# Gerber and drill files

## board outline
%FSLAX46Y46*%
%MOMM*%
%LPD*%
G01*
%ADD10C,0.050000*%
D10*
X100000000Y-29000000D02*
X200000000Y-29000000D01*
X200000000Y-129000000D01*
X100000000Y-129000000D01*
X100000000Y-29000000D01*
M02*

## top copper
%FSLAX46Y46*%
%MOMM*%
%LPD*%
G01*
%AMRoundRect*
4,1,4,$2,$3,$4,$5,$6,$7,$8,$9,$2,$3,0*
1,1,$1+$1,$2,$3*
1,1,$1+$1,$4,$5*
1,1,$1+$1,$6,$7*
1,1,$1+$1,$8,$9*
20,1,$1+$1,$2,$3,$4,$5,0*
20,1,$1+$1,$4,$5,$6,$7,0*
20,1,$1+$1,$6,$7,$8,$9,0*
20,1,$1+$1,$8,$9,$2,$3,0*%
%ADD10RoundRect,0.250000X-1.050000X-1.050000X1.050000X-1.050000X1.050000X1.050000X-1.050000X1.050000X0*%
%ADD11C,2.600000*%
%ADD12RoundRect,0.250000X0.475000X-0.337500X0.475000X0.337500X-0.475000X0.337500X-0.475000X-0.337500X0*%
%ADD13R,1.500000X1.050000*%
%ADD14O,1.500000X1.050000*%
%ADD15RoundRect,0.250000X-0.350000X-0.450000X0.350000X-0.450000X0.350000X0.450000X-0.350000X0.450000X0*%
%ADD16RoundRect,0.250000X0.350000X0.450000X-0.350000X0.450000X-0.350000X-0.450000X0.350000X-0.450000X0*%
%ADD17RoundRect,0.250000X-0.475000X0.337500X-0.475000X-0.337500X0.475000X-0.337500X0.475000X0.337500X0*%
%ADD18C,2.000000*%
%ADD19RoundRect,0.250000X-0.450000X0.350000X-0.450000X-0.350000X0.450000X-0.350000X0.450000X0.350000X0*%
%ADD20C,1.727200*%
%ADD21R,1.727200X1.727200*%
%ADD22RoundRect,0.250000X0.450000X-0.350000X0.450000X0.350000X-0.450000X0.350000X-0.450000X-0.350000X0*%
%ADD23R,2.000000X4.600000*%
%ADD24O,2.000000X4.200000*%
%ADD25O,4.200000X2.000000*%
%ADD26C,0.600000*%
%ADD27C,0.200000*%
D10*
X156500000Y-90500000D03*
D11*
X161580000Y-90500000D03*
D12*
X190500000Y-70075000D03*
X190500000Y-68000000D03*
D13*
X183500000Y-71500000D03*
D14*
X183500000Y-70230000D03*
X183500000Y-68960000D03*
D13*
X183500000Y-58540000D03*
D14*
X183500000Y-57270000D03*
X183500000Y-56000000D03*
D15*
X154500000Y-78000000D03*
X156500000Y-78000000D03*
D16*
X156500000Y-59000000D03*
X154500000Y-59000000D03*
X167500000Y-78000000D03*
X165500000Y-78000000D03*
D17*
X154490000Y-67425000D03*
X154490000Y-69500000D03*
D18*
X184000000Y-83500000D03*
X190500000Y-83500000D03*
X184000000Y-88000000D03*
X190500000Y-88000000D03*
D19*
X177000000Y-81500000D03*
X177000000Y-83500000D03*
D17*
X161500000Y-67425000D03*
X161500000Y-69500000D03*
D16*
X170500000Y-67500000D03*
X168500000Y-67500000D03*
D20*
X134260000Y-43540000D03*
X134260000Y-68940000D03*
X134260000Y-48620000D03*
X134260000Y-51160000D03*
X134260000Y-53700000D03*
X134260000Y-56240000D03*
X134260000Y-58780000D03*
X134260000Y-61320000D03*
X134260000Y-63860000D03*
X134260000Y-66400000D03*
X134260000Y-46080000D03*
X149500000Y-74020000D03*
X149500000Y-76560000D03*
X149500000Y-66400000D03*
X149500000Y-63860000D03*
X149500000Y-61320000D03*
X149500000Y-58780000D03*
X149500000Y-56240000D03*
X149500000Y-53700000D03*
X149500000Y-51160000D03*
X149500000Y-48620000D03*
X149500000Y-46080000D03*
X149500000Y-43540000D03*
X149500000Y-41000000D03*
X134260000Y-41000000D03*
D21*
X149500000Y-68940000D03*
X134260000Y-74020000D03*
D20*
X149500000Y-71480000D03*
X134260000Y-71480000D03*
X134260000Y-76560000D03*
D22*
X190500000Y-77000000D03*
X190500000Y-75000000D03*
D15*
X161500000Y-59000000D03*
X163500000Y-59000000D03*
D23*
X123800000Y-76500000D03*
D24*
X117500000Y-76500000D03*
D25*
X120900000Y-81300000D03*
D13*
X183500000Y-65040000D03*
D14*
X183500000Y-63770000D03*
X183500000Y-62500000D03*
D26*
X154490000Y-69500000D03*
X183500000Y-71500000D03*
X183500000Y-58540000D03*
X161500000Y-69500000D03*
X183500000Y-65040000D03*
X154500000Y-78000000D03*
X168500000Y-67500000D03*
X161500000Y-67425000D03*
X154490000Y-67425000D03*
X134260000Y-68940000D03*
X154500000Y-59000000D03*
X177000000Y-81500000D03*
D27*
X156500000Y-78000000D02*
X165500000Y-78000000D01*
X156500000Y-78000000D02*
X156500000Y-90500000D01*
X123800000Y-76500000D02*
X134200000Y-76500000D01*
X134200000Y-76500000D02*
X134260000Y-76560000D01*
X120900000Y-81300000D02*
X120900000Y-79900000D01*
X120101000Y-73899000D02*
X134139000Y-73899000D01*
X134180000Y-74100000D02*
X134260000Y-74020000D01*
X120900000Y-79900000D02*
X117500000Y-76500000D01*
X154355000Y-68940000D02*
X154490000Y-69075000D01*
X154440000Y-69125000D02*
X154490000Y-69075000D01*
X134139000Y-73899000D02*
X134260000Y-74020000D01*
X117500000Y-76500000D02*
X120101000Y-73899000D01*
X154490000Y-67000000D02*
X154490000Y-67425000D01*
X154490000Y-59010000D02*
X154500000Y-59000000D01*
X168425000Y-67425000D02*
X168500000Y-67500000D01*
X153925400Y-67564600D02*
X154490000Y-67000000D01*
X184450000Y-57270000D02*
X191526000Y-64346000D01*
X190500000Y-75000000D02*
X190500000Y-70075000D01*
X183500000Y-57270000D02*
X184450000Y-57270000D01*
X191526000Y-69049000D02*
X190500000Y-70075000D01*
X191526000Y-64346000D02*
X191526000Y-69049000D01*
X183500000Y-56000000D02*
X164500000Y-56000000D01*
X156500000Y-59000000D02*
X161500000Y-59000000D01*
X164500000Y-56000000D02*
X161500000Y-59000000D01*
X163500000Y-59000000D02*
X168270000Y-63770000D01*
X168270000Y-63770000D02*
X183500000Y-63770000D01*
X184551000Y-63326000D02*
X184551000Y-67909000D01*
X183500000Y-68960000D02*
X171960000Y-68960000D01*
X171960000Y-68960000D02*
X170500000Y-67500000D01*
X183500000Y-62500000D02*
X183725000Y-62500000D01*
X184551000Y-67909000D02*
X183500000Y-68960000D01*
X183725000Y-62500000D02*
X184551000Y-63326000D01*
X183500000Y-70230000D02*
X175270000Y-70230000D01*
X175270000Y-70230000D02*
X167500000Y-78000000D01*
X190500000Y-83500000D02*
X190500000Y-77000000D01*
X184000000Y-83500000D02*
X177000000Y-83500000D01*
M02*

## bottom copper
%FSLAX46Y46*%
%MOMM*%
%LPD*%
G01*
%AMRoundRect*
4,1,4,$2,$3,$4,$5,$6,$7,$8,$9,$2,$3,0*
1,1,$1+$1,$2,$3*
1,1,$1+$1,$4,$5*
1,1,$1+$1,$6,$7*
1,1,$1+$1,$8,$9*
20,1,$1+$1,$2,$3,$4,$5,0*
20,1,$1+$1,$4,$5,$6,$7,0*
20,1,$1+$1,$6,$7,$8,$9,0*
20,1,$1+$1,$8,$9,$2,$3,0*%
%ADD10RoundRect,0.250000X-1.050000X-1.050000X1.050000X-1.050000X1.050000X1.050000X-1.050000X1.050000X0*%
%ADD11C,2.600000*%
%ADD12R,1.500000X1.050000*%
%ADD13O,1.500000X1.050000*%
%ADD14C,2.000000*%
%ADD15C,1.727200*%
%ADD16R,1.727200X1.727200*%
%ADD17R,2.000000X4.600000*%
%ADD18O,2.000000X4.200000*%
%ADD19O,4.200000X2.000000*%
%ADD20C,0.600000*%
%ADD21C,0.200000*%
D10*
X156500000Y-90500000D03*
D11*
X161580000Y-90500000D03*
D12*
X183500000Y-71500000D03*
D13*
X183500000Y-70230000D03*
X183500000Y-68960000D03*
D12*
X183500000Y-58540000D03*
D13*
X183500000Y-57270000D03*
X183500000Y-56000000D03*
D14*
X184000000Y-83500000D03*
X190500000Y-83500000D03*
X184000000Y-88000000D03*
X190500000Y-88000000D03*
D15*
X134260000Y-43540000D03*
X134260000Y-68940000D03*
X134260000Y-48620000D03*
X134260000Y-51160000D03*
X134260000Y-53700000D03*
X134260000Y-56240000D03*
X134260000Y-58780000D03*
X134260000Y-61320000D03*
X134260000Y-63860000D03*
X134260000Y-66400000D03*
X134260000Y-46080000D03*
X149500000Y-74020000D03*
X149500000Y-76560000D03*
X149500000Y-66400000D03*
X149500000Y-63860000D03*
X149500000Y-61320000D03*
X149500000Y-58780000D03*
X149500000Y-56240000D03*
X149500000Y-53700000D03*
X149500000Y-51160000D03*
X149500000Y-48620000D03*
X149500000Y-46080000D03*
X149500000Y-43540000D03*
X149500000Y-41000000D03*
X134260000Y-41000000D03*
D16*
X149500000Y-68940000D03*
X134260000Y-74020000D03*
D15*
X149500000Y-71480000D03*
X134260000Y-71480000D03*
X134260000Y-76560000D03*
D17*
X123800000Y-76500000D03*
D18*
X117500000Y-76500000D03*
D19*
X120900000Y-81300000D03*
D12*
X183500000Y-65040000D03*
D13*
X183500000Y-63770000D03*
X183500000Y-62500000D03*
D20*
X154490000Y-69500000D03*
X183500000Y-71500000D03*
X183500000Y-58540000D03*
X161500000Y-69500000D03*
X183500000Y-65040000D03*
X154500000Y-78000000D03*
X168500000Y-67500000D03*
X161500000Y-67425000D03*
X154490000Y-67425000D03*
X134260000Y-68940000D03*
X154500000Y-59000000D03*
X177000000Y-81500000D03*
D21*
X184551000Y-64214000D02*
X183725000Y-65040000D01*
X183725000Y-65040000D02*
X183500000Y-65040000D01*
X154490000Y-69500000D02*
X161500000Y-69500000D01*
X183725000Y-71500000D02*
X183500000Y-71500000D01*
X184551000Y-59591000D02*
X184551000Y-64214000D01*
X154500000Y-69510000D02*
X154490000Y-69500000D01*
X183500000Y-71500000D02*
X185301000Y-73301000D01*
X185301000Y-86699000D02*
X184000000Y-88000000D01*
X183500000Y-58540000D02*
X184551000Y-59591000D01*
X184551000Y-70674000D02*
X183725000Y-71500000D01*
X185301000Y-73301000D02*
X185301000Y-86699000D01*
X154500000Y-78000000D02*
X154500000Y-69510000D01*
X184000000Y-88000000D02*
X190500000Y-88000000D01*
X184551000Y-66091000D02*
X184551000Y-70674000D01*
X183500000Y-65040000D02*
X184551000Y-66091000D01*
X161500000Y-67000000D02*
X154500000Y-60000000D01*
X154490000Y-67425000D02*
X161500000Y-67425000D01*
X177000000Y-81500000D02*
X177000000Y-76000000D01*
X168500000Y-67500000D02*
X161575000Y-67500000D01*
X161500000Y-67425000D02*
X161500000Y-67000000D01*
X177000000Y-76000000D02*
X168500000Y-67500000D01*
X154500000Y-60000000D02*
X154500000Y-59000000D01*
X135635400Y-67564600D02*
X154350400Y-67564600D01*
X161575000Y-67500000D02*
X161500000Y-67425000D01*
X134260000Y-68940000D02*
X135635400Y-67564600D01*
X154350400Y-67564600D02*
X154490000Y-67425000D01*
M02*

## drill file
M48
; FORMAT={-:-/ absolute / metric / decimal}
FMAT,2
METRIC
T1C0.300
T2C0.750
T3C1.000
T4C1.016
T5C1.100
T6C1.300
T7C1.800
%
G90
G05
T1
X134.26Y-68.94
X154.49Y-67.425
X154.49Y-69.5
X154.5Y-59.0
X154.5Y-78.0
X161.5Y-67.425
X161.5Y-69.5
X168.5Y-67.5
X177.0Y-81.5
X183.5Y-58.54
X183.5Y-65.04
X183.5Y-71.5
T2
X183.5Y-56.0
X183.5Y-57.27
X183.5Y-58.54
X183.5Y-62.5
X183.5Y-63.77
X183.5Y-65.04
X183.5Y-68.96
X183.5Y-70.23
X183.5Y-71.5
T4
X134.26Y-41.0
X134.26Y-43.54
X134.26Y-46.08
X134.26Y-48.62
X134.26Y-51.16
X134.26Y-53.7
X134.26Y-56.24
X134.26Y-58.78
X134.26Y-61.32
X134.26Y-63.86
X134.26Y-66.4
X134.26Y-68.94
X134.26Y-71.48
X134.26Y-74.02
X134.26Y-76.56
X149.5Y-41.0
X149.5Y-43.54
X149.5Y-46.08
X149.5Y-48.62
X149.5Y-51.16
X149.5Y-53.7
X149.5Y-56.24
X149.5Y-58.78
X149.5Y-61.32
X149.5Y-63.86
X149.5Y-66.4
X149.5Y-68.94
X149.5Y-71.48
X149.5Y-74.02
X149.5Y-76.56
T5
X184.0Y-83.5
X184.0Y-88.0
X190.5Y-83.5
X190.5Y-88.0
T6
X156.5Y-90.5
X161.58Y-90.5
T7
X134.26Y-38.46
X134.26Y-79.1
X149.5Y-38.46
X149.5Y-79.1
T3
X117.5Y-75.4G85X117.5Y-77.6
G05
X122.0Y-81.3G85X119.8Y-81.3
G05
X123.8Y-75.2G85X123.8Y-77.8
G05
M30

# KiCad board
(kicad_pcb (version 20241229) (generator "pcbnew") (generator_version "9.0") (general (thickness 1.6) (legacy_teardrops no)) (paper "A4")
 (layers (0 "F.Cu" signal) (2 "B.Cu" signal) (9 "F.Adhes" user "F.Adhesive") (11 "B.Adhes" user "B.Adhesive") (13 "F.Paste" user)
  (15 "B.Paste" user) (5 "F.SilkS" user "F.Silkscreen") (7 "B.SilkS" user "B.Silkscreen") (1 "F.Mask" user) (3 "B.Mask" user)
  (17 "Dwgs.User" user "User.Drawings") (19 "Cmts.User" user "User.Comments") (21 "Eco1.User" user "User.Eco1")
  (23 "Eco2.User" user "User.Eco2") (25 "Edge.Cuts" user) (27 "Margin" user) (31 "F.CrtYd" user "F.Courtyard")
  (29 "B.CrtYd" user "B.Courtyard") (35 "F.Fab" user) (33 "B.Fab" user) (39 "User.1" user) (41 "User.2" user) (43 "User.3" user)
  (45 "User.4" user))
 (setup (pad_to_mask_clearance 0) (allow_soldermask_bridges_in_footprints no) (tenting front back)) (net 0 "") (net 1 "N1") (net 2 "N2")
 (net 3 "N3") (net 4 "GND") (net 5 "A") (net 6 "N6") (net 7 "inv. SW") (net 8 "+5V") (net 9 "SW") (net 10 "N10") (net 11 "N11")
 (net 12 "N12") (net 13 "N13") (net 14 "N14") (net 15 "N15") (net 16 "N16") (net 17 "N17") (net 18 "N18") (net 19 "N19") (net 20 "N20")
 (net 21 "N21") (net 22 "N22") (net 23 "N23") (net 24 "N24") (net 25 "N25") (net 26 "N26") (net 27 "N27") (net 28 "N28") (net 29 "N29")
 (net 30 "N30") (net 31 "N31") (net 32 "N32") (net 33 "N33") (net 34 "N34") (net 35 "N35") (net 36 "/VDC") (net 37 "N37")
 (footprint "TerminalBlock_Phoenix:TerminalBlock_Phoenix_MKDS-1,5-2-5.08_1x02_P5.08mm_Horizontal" (layer "F.Cu") (at 156.5 90.5)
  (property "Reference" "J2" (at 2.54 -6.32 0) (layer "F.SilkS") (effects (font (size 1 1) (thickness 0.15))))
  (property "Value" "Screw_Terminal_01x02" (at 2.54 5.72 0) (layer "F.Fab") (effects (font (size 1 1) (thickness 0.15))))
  (pad "1" thru_hole roundrect (at 0 0) (size 2.6 2.6) (drill 1.3) (layers "*.Cu" "*.Mask") (remove_unused_layers no)
   (roundrect_rratio 0.096154) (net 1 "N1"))
  (pad "2" thru_hole circle (at 5.08 0) (size 2.6 2.6) (drill 1.3) (layers "*.Cu" "*.Mask") (remove_unused_layers no) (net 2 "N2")))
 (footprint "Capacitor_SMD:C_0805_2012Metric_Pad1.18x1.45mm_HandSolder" (layer "F.Cu") (at 190.5 69.0375 90)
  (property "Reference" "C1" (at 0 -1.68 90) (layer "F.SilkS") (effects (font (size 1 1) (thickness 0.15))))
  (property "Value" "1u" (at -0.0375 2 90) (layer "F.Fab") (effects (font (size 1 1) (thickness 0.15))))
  (pad "1" smd roundrect (at -1.0375 0 90) (size 1.175 1.45) (layers "F.Cu" "F.Mask" "F.Paste") (roundrect_rratio 0.212766) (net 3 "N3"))
  (pad "2" smd roundrect (at 1.0375 0 90) (size 1.175 1.45) (layers "F.Cu" "F.Mask" "F.Paste") (roundrect_rratio 0.212766) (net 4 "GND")))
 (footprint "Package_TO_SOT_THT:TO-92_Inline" (layer "F.Cu") (at 183.5 71.5 90)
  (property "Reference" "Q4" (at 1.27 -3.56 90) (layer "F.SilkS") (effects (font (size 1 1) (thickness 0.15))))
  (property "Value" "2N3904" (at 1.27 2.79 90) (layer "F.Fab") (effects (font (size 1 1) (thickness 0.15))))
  (pad "1" thru_hole rect (at 0 0 90) (size 1.05 1.5) (drill 0.75) (layers "*.Cu" "*.Mask") (remove_unused_layers no) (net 4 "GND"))
  (pad "2" thru_hole oval (at 1.27 0 90) (size 1.05 1.5) (drill 0.75) (layers "*.Cu" "*.Mask") (remove_unused_layers no) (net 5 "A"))
  (pad "3" thru_hole oval (at 2.54 0 90) (size 1.05 1.5) (drill 0.75) (layers "*.Cu" "*.Mask") (remove_unused_layers no) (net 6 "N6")))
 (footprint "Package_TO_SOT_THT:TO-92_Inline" (layer "F.Cu") (at 183.5 58.54 90)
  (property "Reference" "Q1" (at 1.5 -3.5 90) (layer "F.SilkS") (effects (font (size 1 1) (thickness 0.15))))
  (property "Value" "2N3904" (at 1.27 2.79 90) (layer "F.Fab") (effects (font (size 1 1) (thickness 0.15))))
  (pad "1" thru_hole rect (at 0 0 90) (size 1.05 1.5) (drill 0.75) (layers "*.Cu" "*.Mask") (remove_unused_layers no) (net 4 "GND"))
  (pad "2" thru_hole oval (at 1.27 0 90) (size 1.05 1.5) (drill 0.75) (layers "*.Cu" "*.Mask") (remove_unused_layers no) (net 3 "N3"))
  (pad "3" thru_hole oval (at 2.54 0 90) (size 1.05 1.5) (drill 0.75) (layers "*.Cu" "*.Mask") (remove_unused_layers no) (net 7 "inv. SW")))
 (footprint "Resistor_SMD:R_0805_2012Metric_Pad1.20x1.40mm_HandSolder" (layer "F.Cu") (at 155.5 78)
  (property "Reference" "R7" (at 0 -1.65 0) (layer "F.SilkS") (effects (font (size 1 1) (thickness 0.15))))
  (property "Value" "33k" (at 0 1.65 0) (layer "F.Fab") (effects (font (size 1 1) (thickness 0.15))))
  (pad "1" smd roundrect (at -1 0) (size 1.2 1.4) (layers "F.Cu" "F.Mask" "F.Paste") (roundrect_rratio 0.208333) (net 4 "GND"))
  (pad "2" smd roundrect (at 1 0) (size 1.2 1.4) (layers "F.Cu" "F.Mask" "F.Paste") (roundrect_rratio 0.208333) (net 1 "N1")))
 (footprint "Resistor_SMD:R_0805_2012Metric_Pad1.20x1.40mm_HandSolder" (layer "F.Cu") (at 155.5 59 180)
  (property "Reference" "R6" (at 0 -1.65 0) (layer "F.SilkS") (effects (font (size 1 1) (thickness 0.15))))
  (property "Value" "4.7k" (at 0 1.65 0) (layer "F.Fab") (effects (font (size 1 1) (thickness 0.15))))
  (pad "1" smd roundrect (at -1 0 180) (size 1.2 1.4) (layers "F.Cu" "F.Mask" "F.Paste") (roundrect_rratio 0.208333) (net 7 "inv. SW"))
  (pad "2" smd roundrect (at 1 0 180) (size 1.2 1.4) (layers "F.Cu" "F.Mask" "F.Paste") (roundrect_rratio 0.208333) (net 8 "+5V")))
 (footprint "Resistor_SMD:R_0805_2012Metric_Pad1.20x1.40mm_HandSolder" (layer "F.Cu") (at 166.5 78 180)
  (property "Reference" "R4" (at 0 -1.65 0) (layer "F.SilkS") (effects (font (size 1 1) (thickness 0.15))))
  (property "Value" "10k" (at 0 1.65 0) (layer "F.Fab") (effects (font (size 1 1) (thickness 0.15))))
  (pad "1" smd roundrect (at -1 0 180) (size 1.2 1.4) (layers "F.Cu" "F.Mask" "F.Paste") (roundrect_rratio 0.208333) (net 5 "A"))
  (pad "2" smd roundrect (at 1 0 180) (size 1.2 1.4) (layers "F.Cu" "F.Mask" "F.Paste") (roundrect_rratio 0.208333) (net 1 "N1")))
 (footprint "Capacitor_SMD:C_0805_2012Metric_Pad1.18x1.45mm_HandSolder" (layer "F.Cu") (at 154.49 68.4625 -90)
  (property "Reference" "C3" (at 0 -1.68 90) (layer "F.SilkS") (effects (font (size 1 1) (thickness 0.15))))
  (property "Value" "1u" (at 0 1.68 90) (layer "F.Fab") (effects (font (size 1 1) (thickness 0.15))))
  (pad "1" smd roundrect (at -1.0375 0 270) (size 1.175 1.45) (layers "F.Cu" "F.Mask" "F.Paste") (roundrect_rratio 0.212766) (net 8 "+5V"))
  (pad "2" smd roundrect (at 1.0375 0 270) (size 1.175 1.45) (layers "F.Cu" "F.Mask" "F.Paste") (roundrect_rratio 0.212766) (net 4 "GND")))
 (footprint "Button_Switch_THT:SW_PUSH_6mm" (layer "F.Cu") (at 184 83.5)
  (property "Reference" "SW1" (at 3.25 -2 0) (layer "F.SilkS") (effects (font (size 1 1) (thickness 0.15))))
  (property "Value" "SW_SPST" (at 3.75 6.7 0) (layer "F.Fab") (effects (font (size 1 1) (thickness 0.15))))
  (pad "1" thru_hole circle (at 0 0 90) (size 2 2) (drill 1.1) (layers "*.Cu" "*.Mask") (remove_unused_layers no) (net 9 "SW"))
  (pad "1" thru_hole circle (at 6.5 0 90) (size 2 2) (drill 1.1) (layers "*.Cu" "*.Mask") (remove_unused_layers no) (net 9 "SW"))
  (pad "2" thru_hole circle (at 0 4.5 90) (size 2 2) (drill 1.1) (layers "*.Cu" "*.Mask") (remove_unused_layers no) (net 4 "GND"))
  (pad "2" thru_hole circle (at 6.5 4.5 90) (size 2 2) (drill 1.1) (layers "*.Cu" "*.Mask") (remove_unused_layers no) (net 4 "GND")))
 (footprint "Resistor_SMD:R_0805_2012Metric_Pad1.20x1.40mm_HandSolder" (layer "F.Cu") (at 177 82.5 -90)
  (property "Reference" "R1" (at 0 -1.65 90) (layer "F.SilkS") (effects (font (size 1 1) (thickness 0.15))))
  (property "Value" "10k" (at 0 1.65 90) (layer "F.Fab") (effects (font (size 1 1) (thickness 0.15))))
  (pad "1" smd roundrect (at -1 0 270) (size 1.2 1.4) (layers "F.Cu" "F.Mask" "F.Paste") (roundrect_rratio 0.208333) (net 8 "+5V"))
  (pad "2" smd roundrect (at 1 0 270) (size 1.2 1.4) (layers "F.Cu" "F.Mask" "F.Paste") (roundrect_rratio 0.208333) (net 9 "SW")))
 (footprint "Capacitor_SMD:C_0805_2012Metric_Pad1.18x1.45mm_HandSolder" (layer "F.Cu") (at 161.5 68.4625 -90)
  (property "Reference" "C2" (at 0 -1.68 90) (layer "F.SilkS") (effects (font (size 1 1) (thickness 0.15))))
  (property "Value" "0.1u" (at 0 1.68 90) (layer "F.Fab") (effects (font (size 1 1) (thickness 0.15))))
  (pad "1" smd roundrect (at -1.0375 0 270) (size 1.175 1.45) (layers "F.Cu" "F.Mask" "F.Paste") (roundrect_rratio 0.212766) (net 8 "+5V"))
  (pad "2" smd roundrect (at 1.0375 0 270) (size 1.175 1.45) (layers "F.Cu" "F.Mask" "F.Paste") (roundrect_rratio 0.212766) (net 4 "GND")))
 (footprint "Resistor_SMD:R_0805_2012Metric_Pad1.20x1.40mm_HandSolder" (layer "F.Cu") (at 169.5 67.5 180)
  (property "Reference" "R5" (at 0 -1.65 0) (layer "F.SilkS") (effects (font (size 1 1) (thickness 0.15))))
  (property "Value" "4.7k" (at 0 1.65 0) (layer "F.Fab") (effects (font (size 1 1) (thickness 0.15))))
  (pad "1" smd roundrect (at -1 0 180) (size 1.2 1.4) (layers "F.Cu" "F.Mask" "F.Paste") (roundrect_rratio 0.208333) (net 6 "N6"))
  (pad "2" smd roundrect (at 1 0 180) (size 1.2 1.4) (layers "F.Cu" "F.Mask" "F.Paste") (roundrect_rratio 0.208333) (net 8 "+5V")))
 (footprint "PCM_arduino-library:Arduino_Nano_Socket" (layer "F.Cu") (at 141.88 37.19 180)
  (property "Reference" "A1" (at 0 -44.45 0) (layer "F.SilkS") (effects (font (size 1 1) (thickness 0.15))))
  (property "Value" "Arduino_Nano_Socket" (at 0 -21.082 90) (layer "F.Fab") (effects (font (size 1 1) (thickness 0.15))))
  (pad "" np_thru_hole circle (at -7.62 -41.91 180) (size 1.8 1.8) (drill 1.8) (layers "*.Cu" "*.Mask"))
  (pad "" np_thru_hole circle (at -7.62 -1.27 180) (size 1.8 1.8) (drill 1.8) (layers "*.Cu" "*.Mask"))
  (pad "" np_thru_hole circle (at 7.62 -41.91 180) (size 1.8 1.8) (drill 1.8) (layers "*.Cu" "*.Mask"))
  (pad "" np_thru_hole circle (at 7.62 -1.27 180) (size 1.8 1.8) (drill 1.8) (layers "*.Cu" "*.Mask"))
  (pad "3V3" thru_hole circle (at 7.62 -6.35 180) (size 1.7272 1.7272) (drill 1.016) (layers "*.Cu" "*.Mask") (remove_unused_layers no)
   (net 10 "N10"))
  (pad "5V" thru_hole circle (at 7.62 -31.75 180) (size 1.7272 1.7272) (drill 1.016) (layers "*.Cu" "*.Mask") (remove_unused_layers no)
   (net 8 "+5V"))
  (pad "A0" thru_hole circle (at 7.62 -11.43 180) (size 1.7272 1.7272) (drill 1.016) (layers "*.Cu" "*.Mask") (remove_unused_layers no)
   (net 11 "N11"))
  (pad "A1" thru_hole circle (at 7.62 -13.97 180) (size 1.7272 1.7272) (drill 1.016) (layers "*.Cu" "*.Mask") (remove_unused_layers no)
   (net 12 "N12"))
  (pad "A2" thru_hole circle (at 7.62 -16.51 180) (size 1.7272 1.7272) (drill 1.016) (layers "*.Cu" "*.Mask") (remove_unused_layers no)
   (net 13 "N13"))
  (pad "A3" thru_hole circle (at 7.62 -19.05 180) (size 1.7272 1.7272) (drill 1.016) (layers "*.Cu" "*.Mask") (remove_unused_layers no)
   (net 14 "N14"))
  (pad "A4" thru_hole circle (at 7.62 -21.59 180) (size 1.7272 1.7272) (drill 1.016) (layers "*.Cu" "*.Mask") (remove_unused_layers no)
   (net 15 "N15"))
  (pad "A5" thru_hole circle (at 7.62 -24.13 180) (size 1.7272 1.7272) (drill 1.016) (layers "*.Cu" "*.Mask") (remove_unused_layers no)
   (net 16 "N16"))
  (pad "A6" thru_hole circle (at 7.62 -26.67 180) (size 1.7272 1.7272) (drill 1.016) (layers "*.Cu" "*.Mask") (remove_unused_layers no)
   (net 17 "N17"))
  (pad "A7" thru_hole circle (at 7.62 -29.21 180) (size 1.7272 1.7272) (drill 1.016) (layers "*.Cu" "*.Mask") (remove_unused_layers no)
   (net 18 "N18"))
  (pad "AREF" thru_hole circle (at 7.62 -8.89 180) (size 1.7272 1.7272) (drill 1.016) (layers "*.Cu" "*.Mask") (remove_unused_layers no)
   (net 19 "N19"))
  (pad "D0" thru_hole circle (at -7.62 -36.83 180) (size 1.7272 1.7272) (drill 1.016) (layers "*.Cu" "*.Mask") (remove_unused_layers no)
   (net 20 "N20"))
  (pad "D1" thru_hole circle (at -7.62 -39.37 180) (size 1.7272 1.7272) (drill 1.016) (layers "*.Cu" "*.Mask") (remove_unused_layers no)
   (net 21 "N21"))
  (pad "D2" thru_hole circle (at -7.62 -29.21 180) (size 1.7272 1.7272) (drill 1.016) (layers "*.Cu" "*.Mask") (remove_unused_layers no)
   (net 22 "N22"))
  (pad "D3" thru_hole circle (at -7.62 -26.67 180) (size 1.7272 1.7272) (drill 1.016) (layers "*.Cu" "*.Mask") (remove_unused_layers no)
   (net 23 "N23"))
  (pad "D4" thru_hole circle (at -7.62 -24.13 180) (size 1.7272 1.7272) (drill 1.016) (layers "*.Cu" "*.Mask") (remove_unused_layers no)
   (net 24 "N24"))
  (pad "D5" thru_hole circle (at -7.62 -21.59 180) (size 1.7272 1.7272) (drill 1.016) (layers "*.Cu" "*.Mask") (remove_unused_layers no)
   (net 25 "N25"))
  (pad "D6" thru_hole circle (at -7.62 -19.05 180) (size 1.7272 1.7272) (drill 1.016) (layers "*.Cu" "*.Mask") (remove_unused_layers no)
   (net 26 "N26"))
  (pad "D7" thru_hole circle (at -7.62 -16.51 180) (size 1.7272 1.7272) (drill 1.016) (layers "*.Cu" "*.Mask") (remove_unused_layers no)
   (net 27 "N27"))
  (pad "D8" thru_hole circle (at -7.62 -13.97 180) (size 1.7272 1.7272) (drill 1.016) (layers "*.Cu" "*.Mask") (remove_unused_layers no)
   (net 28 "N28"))
  (pad "D9" thru_hole circle (at -7.62 -11.43 180) (size 1.7272 1.7272) (drill 1.016) (layers "*.Cu" "*.Mask") (remove_unused_layers no)
   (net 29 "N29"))
  (pad "D10" thru_hole circle (at -7.62 -8.89 180) (size 1.7272 1.7272) (drill 1.016) (layers "*.Cu" "*.Mask") (remove_unused_layers no)
   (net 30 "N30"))
  (pad "D11" thru_hole circle (at -7.62 -6.35 180) (size 1.7272 1.7272) (drill 1.016) (layers "*.Cu" "*.Mask") (remove_unused_layers no)
   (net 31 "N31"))
  (pad "D12" thru_hole circle (at -7.62 -3.81 180) (size 1.7272 1.7272) (drill 1.016) (layers "*.Cu" "*.Mask") (remove_unused_layers no)
   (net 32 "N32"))
  (pad "D13" thru_hole circle (at 7.62 -3.81 180) (size 1.7272 1.7272) (drill 1.016) (layers "*.Cu" "*.Mask") (remove_unused_layers no)
   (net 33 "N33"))
  (pad "GND1" thru_hole rect (at -7.62 -31.75 180) (size 1.7272 1.7272) (drill 1.016) (layers "*.Cu" "*.Mask") (remove_unused_layers no)
   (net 4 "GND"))
  (pad "GND2" thru_hole rect (at 7.62 -36.83 180) (size 1.7272 1.7272) (drill 1.016) (layers "*.Cu" "*.Mask") (remove_unused_layers no)
   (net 4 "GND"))
  (pad "RST1" thru_hole circle (at -7.62 -34.29 180) (size 1.7272 1.7272) (drill 1.016) (layers "*.Cu" "*.Mask") (remove_unused_layers no)
   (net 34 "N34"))
  (pad "RST2" thru_hole circle (at 7.62 -34.29 180) (size 1.7272 1.7272) (drill 1.016) (layers "*.Cu" "*.Mask") (remove_unused_layers no)
   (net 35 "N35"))
  (pad "VIN" thru_hole circle (at 7.62 -39.37 180) (size 1.7272 1.7272) (drill 1.016) (layers "*.Cu" "*.Mask") (remove_unused_layers no)
   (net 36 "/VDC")))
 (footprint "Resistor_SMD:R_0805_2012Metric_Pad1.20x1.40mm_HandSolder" (layer "F.Cu") (at 190.5 76 90)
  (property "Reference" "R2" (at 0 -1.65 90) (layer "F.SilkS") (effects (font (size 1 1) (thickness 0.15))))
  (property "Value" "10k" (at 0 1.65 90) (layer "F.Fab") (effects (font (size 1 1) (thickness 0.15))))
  (pad "1" smd roundrect (at -1 0 90) (size 1.2 1.4) (layers "F.Cu" "F.Mask" "F.Paste") (roundrect_rratio 0.208333) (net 9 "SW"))
  (pad "2" smd roundrect (at 1 0 90) (size 1.2 1.4) (layers "F.Cu" "F.Mask" "F.Paste") (roundrect_rratio 0.208333) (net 3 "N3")))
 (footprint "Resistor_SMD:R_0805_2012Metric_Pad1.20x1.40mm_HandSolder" (layer "F.Cu") (at 162.5 59)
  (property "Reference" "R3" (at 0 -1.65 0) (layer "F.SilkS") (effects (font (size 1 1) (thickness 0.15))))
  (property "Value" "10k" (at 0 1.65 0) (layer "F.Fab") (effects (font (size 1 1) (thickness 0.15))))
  (pad "1" smd roundrect (at -1 0) (size 1.2 1.4) (layers "F.Cu" "F.Mask" "F.Paste") (roundrect_rratio 0.208333) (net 7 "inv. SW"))
  (pad "2" smd roundrect (at 1 0) (size 1.2 1.4) (layers "F.Cu" "F.Mask" "F.Paste") (roundrect_rratio 0.208333) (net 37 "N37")))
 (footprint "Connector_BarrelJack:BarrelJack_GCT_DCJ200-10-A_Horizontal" (layer "F.Cu") (at 123.8 76.5 -90)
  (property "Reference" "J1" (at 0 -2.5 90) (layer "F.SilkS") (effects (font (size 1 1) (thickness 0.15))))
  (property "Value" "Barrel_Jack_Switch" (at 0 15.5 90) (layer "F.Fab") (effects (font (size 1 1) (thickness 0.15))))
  (pad "1" thru_hole rect (at 0 0 270) (size 4.6 2) (drill oval 3.6 1) (layers "*.Cu" "*.Mask") (remove_unused_layers no) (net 36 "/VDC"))
  (pad "2" thru_hole oval (at 0 6.3 270) (size 4.2 2) (drill oval 3.2 1) (layers "*.Cu" "*.Mask") (remove_unused_layers no) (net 4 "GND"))
  (pad "3" thru_hole oval (at 4.8 2.9 270) (size 2 4.2) (drill oval 1 3.2) (layers "*.Cu" "*.Mask") (remove_unused_layers no) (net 4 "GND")))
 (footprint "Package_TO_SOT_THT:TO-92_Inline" (layer "F.Cu") (at 183.5 65.04 90)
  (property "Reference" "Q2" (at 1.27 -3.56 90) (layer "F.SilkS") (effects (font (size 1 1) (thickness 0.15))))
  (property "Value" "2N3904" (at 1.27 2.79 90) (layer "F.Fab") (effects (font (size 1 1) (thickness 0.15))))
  (pad "1" thru_hole rect (at 0 0 90) (size 1.05 1.5) (drill 0.75) (layers "*.Cu" "*.Mask") (remove_unused_layers no) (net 4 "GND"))
  (pad "2" thru_hole oval (at 1.27 0 90) (size 1.05 1.5) (drill 0.75) (layers "*.Cu" "*.Mask") (remove_unused_layers no) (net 37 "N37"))
  (pad "3" thru_hole oval (at 2.54 0 90) (size 1.05 1.5) (drill 0.75) (layers "*.Cu" "*.Mask") (remove_unused_layers no) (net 6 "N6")))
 (gr_rect (start 100 29) (end 200 129) (stroke (width 0.05) (type default)) (fill no) (layer "Edge.Cuts"))
 (segment (start 156.5 78) (end 165.5 78) (width 0.2) (layer "F.Cu") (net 1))
 (segment (start 156.5 78) (end 156.5 90.5) (width 0.2) (layer "F.Cu") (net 1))
 (segment (start 123.8 76.5) (end 134.2 76.5) (width 0.2) (layer "F.Cu") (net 36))
 (segment (start 134.2 76.5) (end 134.26 76.56) (width 0.2) (layer "F.Cu") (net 36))
 (segment (start 120.9 81.3) (end 120.9 79.9) (width 0.2) (layer "F.Cu") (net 4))
 (segment (start 120.101 73.899) (end 134.139 73.899) (width 0.2) (layer "F.Cu") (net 4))
 (segment (start 134.18 74.1) (end 134.26 74.02) (width 0.2) (layer "F.Cu") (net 4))
 (segment (start 120.9 79.9) (end 117.5 76.5) (width 0.2) (layer "F.Cu") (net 4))
 (segment (start 154.355 68.94) (end 154.49 69.075) (width 0.2) (layer "F.Cu") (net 4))
 (segment (start 154.44 69.125) (end 154.49 69.075) (width 0.2) (layer "F.Cu") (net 4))
 (segment (start 134.139 73.899) (end 134.26 74.02) (width 0.2) (layer "F.Cu") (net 4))
 (segment (start 117.5 76.5) (end 120.101 73.899) (width 0.2) (layer "F.Cu") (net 4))
 (via (at 154.49 69.5) (size 0.6) (drill 0.3) (layers "F.Cu" "B.Cu") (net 4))
 (via (at 183.5 71.5) (size 0.6) (drill 0.3) (layers "F.Cu" "B.Cu") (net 4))
 (via (at 183.5 58.54) (size 0.6) (drill 0.3) (layers "F.Cu" "B.Cu") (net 4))
 (via (at 161.5 69.5) (size 0.6) (drill 0.3) (layers "F.Cu" "B.Cu") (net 4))
 (via (at 183.5 65.04) (size 0.6) (drill 0.3) (layers "F.Cu" "B.Cu") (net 4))
 (via (at 154.5 78) (size 0.6) (drill 0.3) (layers "F.Cu" "B.Cu") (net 4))
 (segment (start 184.551 64.214) (end 183.725 65.04) (width 0.2) (layer "B.Cu") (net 4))
 (segment (start 183.725 65.04) (end 183.5 65.04) (width 0.2) (layer "B.Cu") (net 4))
 (segment (start 154.49 69.5) (end 161.5 69.5) (width 0.2) (layer "B.Cu") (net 4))
 (segment (start 183.725 71.5) (end 183.5 71.5) (width 0.2) (layer "B.Cu") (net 4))
 (segment (start 184.551 59.591) (end 184.551 64.214) (width 0.2) (layer "B.Cu") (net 4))
 (segment (start 154.5 69.51) (end 154.49 69.5) (width 0.2) (layer "B.Cu") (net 4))
 (segment (start 183.5 71.5) (end 185.301 73.301) (width 0.2) (layer "B.Cu") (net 4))
 (segment (start 185.301 86.699) (end 184 88) (width 0.2) (layer "B.Cu") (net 4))
 (segment (start 183.5 58.54) (end 184.551 59.591) (width 0.2) (layer "B.Cu") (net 4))
 (segment (start 184.551 70.674) (end 183.725 71.5) (width 0.2) (layer "B.Cu") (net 4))
 (segment (start 185.301 73.301) (end 185.301 86.699) (width 0.2) (layer "B.Cu") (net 4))
 (segment (start 154.5 78) (end 154.5 69.51) (width 0.2) (layer "B.Cu") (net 4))
 (segment (start 184 88) (end 190.5 88) (width 0.2) (layer "B.Cu") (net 4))
 (segment (start 184.551 66.091) (end 184.551 70.674) (width 0.2) (layer "B.Cu") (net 4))
 (segment (start 183.5 65.04) (end 184.551 66.091) (width 0.2) (layer "B.Cu") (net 4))
 (segment (start 154.49 67) (end 154.49 67.425) (width 0.2) (layer "F.Cu") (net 8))
 (segment (start 154.49 59.01) (end 154.5 59) (width 0.2) (layer "F.Cu") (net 8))
 (segment (start 168.425 67.425) (end 168.5 67.5) (width 0.2) (layer "F.Cu") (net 8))
 (segment (start 153.9254 67.5646) (end 154.49 67) (width 0.2) (layer "F.Cu") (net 8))
 (via (at 168.5 67.5) (size 0.6) (drill 0.3) (layers "F.Cu" "B.Cu") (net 8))
 (via (at 161.5 67.425) (size 0.6) (drill 0.3) (layers "F.Cu" "B.Cu") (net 8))
 (via (at 154.49 67.425) (size 0.6) (drill 0.3) (layers "F.Cu" "B.Cu") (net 8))
 (via (at 134.26 68.94) (size 0.6) (drill 0.3) (layers "F.Cu" "B.Cu") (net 8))
 (via (at 154.5 59) (size 0.6) (drill 0.3) (layers "F.Cu" "B.Cu") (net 8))
 (via (at 177 81.5) (size 0.6) (drill 0.3) (layers "F.Cu" "B.Cu") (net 8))
 (segment (start 161.5 67) (end 154.5 60) (width 0.2) (layer "B.Cu") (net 8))
 (segment (start 154.49 67.425) (end 161.5 67.425) (width 0.2) (layer "B.Cu") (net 8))
 (segment (start 177 81.5) (end 177 76) (width 0.2) (layer "B.Cu") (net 8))
 (segment (start 168.5 67.5) (end 161.575 67.5) (width 0.2) (layer "B.Cu") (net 8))
 (segment (start 161.5 67.425) (end 161.5 67) (width 0.2) (layer "B.Cu") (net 8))
 (segment (start 177 76) (end 168.5 67.5) (width 0.2) (layer "B.Cu") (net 8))
 (segment (start 154.5 60) (end 154.5 59) (width 0.2) (layer "B.Cu") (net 8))
 (segment (start 135.6354 67.5646) (end 154.3504 67.5646) (width 0.2) (layer "B.Cu") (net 8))
 (segment (start 161.575 67.5) (end 161.5 67.425) (width 0.2) (layer "B.Cu") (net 8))
 (segment (start 134.26 68.94) (end 135.6354 67.5646) (width 0.2) (layer "B.Cu") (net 8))
 (segment (start 154.3504 67.5646) (end 154.49 67.425) (width 0.2) (layer "B.Cu") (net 8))
 (segment (start 184.45 57.27) (end 191.526 64.346) (width 0.2) (layer "F.Cu") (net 3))
 (segment (start 190.5 75) (end 190.5 70.075) (width 0.2) (layer "F.Cu") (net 3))
 (segment (start 183.5 57.27) (end 184.45 57.27) (width 0.2) (layer "F.Cu") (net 3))
 (segment (start 191.526 69.049) (end 190.5 70.075) (width 0.2) (layer "F.Cu") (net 3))
 (segment (start 191.526 64.346) (end 191.526 69.049) (width 0.2) (layer "F.Cu") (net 3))
 (segment (start 183.5 56) (end 164.5 56) (width 0.2) (layer "F.Cu") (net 7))
 (segment (start 156.5 59) (end 161.5 59) (width 0.2) (layer "F.Cu") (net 7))
 (segment (start 164.5 56) (end 161.5 59) (width 0.2) (layer "F.Cu") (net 7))
 (segment (start 163.5 59) (end 168.27 63.77) (width 0.2) (layer "F.Cu") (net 37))
 (segment (start 168.27 63.77) (end 183.5 63.77) (width 0.2) (layer "F.Cu") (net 37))
 (segment (start 184.551 63.326) (end 184.551 67.909) (width 0.2) (layer "F.Cu") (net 6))
 (segment (start 183.5 68.96) (end 171.96 68.96) (width 0.2) (layer "F.Cu") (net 6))
 (segment (start 171.96 68.96) (end 170.5 67.5) (width 0.2) (layer "F.Cu") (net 6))
 (segment (start 183.5 62.5) (end 183.725 62.5) (width 0.2) (layer "F.Cu") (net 6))
 (segment (start 184.551 67.909) (end 183.5 68.96) (width 0.2) (layer "F.Cu") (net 6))
 (segment (start 183.725 62.5) (end 184.551 63.326) (width 0.2) (layer "F.Cu") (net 6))
 (segment (start 183.5 70.23) (end 175.27 70.23) (width 0.2) (layer "F.Cu") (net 5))
 (segment (start 175.27 70.23) (end 167.5 78) (width 0.2) (layer "F.Cu") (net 5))
 (segment (start 190.5 83.5) (end 190.5 77) (width 0.2) (layer "F.Cu") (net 9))
 (segment (start 184 83.5) (end 177 83.5) (width 0.2) (layer "F.Cu") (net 9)))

